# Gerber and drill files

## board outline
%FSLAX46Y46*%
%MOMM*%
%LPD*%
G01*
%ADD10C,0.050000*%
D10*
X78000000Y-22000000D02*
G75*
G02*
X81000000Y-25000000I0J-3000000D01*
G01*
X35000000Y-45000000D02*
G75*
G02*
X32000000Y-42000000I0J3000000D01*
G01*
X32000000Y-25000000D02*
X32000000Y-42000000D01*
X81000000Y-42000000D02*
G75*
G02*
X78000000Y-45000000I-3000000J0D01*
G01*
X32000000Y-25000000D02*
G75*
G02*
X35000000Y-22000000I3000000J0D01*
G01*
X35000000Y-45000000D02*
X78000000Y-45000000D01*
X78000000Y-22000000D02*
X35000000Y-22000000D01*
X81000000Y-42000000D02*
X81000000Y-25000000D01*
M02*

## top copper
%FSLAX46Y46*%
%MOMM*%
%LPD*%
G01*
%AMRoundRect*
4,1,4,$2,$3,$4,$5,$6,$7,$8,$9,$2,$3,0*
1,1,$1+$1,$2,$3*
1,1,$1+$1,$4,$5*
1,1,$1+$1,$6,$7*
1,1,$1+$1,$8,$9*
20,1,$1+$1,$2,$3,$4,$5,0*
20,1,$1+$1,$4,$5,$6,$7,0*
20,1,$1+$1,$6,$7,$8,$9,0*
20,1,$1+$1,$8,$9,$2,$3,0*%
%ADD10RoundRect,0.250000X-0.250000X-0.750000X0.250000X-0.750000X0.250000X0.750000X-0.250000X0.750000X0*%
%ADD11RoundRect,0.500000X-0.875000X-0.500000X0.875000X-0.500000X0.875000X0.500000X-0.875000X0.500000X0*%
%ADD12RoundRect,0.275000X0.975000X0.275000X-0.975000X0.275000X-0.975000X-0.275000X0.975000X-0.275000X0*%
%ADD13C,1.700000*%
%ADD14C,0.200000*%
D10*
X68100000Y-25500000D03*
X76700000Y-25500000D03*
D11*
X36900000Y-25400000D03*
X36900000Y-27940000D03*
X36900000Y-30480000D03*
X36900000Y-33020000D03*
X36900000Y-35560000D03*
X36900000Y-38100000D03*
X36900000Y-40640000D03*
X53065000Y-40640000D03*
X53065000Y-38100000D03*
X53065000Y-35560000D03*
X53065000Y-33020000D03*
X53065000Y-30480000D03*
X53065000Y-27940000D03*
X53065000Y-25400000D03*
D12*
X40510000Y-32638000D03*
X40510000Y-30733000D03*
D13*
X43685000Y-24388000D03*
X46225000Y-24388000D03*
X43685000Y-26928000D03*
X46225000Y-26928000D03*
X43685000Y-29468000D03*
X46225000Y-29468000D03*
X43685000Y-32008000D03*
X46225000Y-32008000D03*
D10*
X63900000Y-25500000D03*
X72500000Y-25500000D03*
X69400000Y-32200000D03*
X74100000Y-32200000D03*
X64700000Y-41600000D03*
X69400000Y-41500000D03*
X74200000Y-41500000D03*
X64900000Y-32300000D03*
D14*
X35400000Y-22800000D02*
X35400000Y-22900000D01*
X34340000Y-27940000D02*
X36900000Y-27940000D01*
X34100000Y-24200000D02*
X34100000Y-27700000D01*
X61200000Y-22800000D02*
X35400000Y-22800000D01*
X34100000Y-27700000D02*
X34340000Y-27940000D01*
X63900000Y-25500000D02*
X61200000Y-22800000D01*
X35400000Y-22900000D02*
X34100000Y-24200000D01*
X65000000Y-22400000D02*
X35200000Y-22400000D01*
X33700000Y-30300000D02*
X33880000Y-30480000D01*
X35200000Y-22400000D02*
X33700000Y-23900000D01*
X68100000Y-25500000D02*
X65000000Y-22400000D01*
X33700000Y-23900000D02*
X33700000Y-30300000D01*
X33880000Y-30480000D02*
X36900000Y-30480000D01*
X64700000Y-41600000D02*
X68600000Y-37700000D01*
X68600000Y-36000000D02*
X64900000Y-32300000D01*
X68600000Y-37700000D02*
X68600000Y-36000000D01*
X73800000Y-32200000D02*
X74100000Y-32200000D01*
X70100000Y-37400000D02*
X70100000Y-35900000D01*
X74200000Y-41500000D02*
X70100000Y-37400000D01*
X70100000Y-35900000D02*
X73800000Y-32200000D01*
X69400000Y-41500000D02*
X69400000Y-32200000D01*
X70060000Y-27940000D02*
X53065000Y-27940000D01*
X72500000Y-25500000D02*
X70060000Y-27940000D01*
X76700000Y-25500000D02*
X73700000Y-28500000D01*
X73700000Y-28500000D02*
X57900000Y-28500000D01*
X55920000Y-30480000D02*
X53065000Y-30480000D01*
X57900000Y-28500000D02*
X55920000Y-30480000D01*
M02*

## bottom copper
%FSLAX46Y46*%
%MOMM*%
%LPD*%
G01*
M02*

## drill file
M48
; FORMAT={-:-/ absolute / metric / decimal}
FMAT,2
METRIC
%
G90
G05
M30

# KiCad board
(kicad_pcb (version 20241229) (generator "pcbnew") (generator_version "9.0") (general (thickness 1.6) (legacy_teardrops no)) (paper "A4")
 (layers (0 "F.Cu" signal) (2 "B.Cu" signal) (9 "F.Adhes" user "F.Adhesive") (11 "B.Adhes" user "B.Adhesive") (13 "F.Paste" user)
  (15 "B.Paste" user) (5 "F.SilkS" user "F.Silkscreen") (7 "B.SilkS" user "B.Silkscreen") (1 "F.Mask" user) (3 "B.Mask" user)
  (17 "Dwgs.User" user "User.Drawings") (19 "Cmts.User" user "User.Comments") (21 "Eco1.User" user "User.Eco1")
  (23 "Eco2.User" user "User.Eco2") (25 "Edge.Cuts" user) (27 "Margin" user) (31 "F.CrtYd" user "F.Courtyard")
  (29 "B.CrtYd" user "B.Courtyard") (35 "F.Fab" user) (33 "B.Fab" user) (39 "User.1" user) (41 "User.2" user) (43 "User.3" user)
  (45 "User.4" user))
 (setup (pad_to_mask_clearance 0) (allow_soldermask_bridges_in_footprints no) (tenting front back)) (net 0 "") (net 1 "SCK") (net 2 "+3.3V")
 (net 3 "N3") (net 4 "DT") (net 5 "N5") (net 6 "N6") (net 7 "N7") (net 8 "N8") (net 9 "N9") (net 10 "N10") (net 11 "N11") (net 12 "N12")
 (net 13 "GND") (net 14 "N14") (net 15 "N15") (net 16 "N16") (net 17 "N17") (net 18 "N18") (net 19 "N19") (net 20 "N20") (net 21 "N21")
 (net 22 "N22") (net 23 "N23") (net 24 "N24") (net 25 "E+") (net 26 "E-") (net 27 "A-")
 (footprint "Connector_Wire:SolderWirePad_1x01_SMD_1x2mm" (layer "F.Cu") (at 68.1 25.5)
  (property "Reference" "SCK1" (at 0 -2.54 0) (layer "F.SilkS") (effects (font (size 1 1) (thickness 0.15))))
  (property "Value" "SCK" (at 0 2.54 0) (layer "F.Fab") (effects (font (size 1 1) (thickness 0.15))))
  (pad "1" smd roundrect (at 0 0) (size 1 2) (layers "F.Cu" "F.Mask" "F.Paste") (roundrect_rratio 0.25) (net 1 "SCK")))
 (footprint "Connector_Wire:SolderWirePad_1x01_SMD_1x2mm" (layer "F.Cu") (at 76.7 25.5)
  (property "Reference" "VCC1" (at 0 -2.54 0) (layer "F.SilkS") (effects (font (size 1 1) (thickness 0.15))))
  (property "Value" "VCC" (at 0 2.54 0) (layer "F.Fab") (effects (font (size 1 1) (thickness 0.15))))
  (pad "1" smd roundrect (at 0 0) (size 1 2) (layers "F.Cu" "F.Mask" "F.Paste") (roundrect_rratio 0.25) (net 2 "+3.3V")))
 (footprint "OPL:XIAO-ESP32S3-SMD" (layer "F.Cu") (at 44.961364 32.973)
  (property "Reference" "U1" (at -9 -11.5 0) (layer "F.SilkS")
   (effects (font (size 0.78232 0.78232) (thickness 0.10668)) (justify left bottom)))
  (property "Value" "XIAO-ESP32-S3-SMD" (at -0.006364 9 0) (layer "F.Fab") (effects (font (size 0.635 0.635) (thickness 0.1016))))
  (pad "1" smd roundrect (at -8.061364 -7.573) (size 2.75 2) (layers "F.Cu" "F.Mask" "F.Paste") (roundrect_rratio 0.25) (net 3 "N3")
   (solder_mask_margin 0.0508) (thermal_bridge_angle 45))
  (pad "2" smd roundrect (at -8.061364 -5.033) (size 2.75 2) (layers "F.Cu" "F.Mask" "F.Paste") (roundrect_rratio 0.25) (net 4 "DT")
   (solder_mask_margin 0.0508) (thermal_bridge_angle 45))
  (pad "3" smd roundrect (at -8.061364 -2.493) (size 2.75 2) (layers "F.Cu" "F.Mask" "F.Paste") (roundrect_rratio 0.25) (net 1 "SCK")
   (solder_mask_margin 0.0508) (thermal_bridge_angle 45))
  (pad "4" smd roundrect (at -8.061364 0.047) (size 2.75 2) (layers "F.Cu" "F.Mask" "F.Paste") (roundrect_rratio 0.25) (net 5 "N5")
   (solder_mask_margin 0.0508) (thermal_bridge_angle 45))
  (pad "5" smd roundrect (at -8.061364 2.587) (size 2.75 2) (layers "F.Cu" "F.Mask" "F.Paste") (roundrect_rratio 0.25) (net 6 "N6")
   (solder_mask_margin 0.0508) (thermal_bridge_angle 45))
  (pad "6" smd roundrect (at -8.061364 5.127) (size 2.75 2) (layers "F.Cu" "F.Mask" "F.Paste") (roundrect_rratio 0.25) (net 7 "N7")
   (solder_mask_margin 0.0508) (thermal_bridge_angle 45))
  (pad "7" smd roundrect (at -8.061364 7.667) (size 2.75 2) (layers "F.Cu" "F.Mask" "F.Paste") (roundrect_rratio 0.25) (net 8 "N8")
   (solder_mask_margin 0.0508) (thermal_bridge_angle 45))
  (pad "8" smd roundrect (at 8.103636 7.667) (size 2.75 2) (layers "F.Cu" "F.Mask" "F.Paste") (roundrect_rratio 0.25) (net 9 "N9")
   (solder_mask_margin 0.0508) (thermal_bridge_angle 45))
  (pad "9" smd roundrect (at 8.103636 5.127) (size 2.75 2) (layers "F.Cu" "F.Mask" "F.Paste") (roundrect_rratio 0.25) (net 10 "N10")
   (solder_mask_margin 0.0508) (thermal_bridge_angle 45))
  (pad "10" smd roundrect (at 8.103636 2.587) (size 2.75 2) (layers "F.Cu" "F.Mask" "F.Paste") (roundrect_rratio 0.25) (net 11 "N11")
   (solder_mask_margin 0.0508) (thermal_bridge_angle 45))
  (pad "11" smd roundrect (at 8.103636 0.047) (size 2.75 2) (layers "F.Cu" "F.Mask" "F.Paste") (roundrect_rratio 0.25) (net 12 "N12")
   (solder_mask_margin 0.0508) (thermal_bridge_angle 45))
  (pad "12" smd roundrect (at 8.103636 -2.493) (size 2.75 2) (layers "F.Cu" "F.Mask" "F.Paste") (roundrect_rratio 0.25) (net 2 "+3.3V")
   (solder_mask_margin 0.0508) (thermal_bridge_angle 45))
  (pad "13" smd roundrect (at 8.103636 -5.033) (size 2.75 2) (layers "F.Cu" "F.Mask" "F.Paste") (roundrect_rratio 0.25) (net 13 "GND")
   (solder_mask_margin 0.0508) (thermal_bridge_angle 45))
  (pad "14" smd roundrect (at 8.103636 -7.573) (size 2.75 2) (layers "F.Cu" "F.Mask" "F.Paste") (roundrect_rratio 0.25) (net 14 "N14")
   (solder_mask_margin 0.0508) (thermal_bridge_angle 45))
  (pad "15" smd roundrect (at -4.451364 -0.335 180) (size 2.5 1.1) (layers "F.Cu" "F.Mask" "F.Paste") (roundrect_rratio 0.25) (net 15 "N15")
   (solder_mask_margin 0.0508) (thermal_bridge_angle 45))
  (pad "16" smd roundrect (at -4.451364 -2.24 180) (size 2.5 1.1) (layers "F.Cu" "F.Mask" "F.Paste") (roundrect_rratio 0.25) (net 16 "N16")
   (solder_mask_margin 0.0508) (thermal_bridge_angle 45))
  (pad "17" smd circle (at -1.276364 -8.585) (size 1.7 1.7) (layers "F.Cu" "F.Mask" "F.Paste") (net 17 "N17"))
  (pad "18" smd circle (at 1.263636 -8.585) (size 1.7 1.7) (layers "F.Cu" "F.Mask" "F.Paste") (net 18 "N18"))
  (pad "19" smd circle (at -1.276364 -6.045) (size 1.7 1.7) (layers "F.Cu" "F.Mask" "F.Paste") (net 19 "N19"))
  (pad "20" smd circle (at 1.263636 -6.045) (size 1.7 1.7) (layers "F.Cu" "F.Mask" "F.Paste") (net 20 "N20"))
  (pad "21" smd circle (at -1.276364 -3.505) (size 1.7 1.7) (layers "F.Cu" "F.Mask" "F.Paste") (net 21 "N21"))
  (pad "22" smd circle (at 1.263636 -3.505) (size 1.7 1.7) (layers "F.Cu" "F.Mask" "F.Paste") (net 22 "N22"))
  (pad "23" smd circle (at -1.276364 -0.965) (size 1.7 1.7) (layers "F.Cu" "F.Mask" "F.Paste") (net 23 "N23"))
  (pad "24" smd circle (at 1.263636 -0.965) (size 1.7 1.7) (layers "F.Cu" "F.Mask" "F.Paste") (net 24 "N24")))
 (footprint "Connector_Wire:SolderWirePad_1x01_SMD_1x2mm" (layer "F.Cu") (at 63.9 25.5)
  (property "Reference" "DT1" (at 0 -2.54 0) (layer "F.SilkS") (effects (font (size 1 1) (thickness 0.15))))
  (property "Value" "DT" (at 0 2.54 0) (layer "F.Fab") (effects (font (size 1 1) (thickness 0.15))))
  (pad "1" smd roundrect (at 0 0) (size 1 2) (layers "F.Cu" "F.Mask" "F.Paste") (roundrect_rratio 0.25) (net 4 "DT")))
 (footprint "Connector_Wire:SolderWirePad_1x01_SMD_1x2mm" (layer "F.Cu") (at 72.5 25.5)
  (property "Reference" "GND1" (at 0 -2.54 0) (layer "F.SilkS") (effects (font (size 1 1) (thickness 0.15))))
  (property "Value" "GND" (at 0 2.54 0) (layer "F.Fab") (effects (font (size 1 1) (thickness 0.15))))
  (pad "1" smd roundrect (at 0 0) (size 1 2) (layers "F.Cu" "F.Mask" "F.Paste") (roundrect_rratio 0.25) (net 13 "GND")))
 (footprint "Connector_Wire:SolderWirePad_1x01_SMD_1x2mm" (layer "F.Cu") (at 69.4 32.2)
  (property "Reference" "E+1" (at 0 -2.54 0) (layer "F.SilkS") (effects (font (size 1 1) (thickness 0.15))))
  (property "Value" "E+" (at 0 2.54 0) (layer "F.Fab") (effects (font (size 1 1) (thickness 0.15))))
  (pad "1" smd roundrect (at 0 0) (size 1 2) (layers "F.Cu" "F.Mask" "F.Paste") (roundrect_rratio 0.25) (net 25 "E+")))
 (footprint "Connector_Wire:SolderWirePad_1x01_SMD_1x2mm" (layer "F.Cu") (at 74.1 32.2)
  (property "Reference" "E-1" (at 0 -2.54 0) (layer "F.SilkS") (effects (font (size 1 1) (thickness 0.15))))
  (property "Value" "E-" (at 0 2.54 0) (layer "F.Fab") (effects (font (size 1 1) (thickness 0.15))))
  (pad "1" smd roundrect (at 0 0) (size 1 2) (layers "F.Cu" "F.Mask" "F.Paste") (roundrect_rratio 0.25) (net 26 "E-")))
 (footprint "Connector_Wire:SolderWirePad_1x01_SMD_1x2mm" (layer "F.Cu") (at 64.7 41.6)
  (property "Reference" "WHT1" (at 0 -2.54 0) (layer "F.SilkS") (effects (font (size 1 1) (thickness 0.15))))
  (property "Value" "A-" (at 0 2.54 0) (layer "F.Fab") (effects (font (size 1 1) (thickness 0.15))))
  (pad "1" smd roundrect (at 0 0) (size 1 2) (layers "F.Cu" "F.Mask" "F.Paste") (roundrect_rratio 0.25) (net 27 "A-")))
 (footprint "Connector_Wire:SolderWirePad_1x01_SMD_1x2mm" (layer "F.Cu") (at 69.4 41.5)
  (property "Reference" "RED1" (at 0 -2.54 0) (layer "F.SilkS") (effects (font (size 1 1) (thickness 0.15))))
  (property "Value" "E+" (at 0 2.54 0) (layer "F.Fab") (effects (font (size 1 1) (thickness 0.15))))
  (pad "1" smd roundrect (at 0 0) (size 1 2) (layers "F.Cu" "F.Mask" "F.Paste") (roundrect_rratio 0.25) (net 25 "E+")))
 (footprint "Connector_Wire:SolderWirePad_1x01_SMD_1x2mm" (layer "F.Cu") (at 74.2 41.5)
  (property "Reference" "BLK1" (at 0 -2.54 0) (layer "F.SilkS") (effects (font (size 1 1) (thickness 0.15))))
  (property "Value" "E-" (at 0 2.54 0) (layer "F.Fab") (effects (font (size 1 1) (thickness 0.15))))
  (pad "1" smd roundrect (at 0 0) (size 1 2) (layers "F.Cu" "F.Mask" "F.Paste") (roundrect_rratio 0.25) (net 26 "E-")))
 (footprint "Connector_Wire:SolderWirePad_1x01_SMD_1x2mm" (layer "F.Cu") (at 64.9 32.3)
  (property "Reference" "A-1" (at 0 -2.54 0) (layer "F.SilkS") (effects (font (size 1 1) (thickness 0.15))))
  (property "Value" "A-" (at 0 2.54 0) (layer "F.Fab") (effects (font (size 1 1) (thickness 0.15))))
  (pad "1" smd roundrect (at 0 0) (size 1 2) (layers "F.Cu" "F.Mask" "F.Paste") (roundrect_rratio 0.25) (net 27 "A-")))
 (gr_arc (start 78 22) (mid 80.12132 22.87868) (end 81 25) (stroke (width 0.05) (type default)) (layer "Edge.Cuts"))
 (gr_arc (start 35 45) (mid 32.87868 44.12132) (end 32 42) (stroke (width 0.05) (type default)) (layer "Edge.Cuts"))
 (gr_line (start 32 25) (end 32 42) (stroke (width 0.05) (type default)) (layer "Edge.Cuts"))
 (gr_arc (start 81 42) (mid 80.12132 44.12132) (end 78 45) (stroke (width 0.05) (type default)) (layer "Edge.Cuts"))
 (gr_arc (start 32 25) (mid 32.87868 22.87868) (end 35 22) (stroke (width 0.05) (type default)) (layer "Edge.Cuts"))
 (gr_line (start 35 45) (end 78 45) (stroke (width 0.05) (type default)) (layer "Edge.Cuts"))
 (gr_line (start 78 22) (end 35 22) (stroke (width 0.05) (type default)) (layer "Edge.Cuts"))
 (gr_line (start 81 42) (end 81 25) (stroke (width 0.05) (type default)) (layer "Edge.Cuts"))
 (segment (start 35.4 22.8) (end 35.4 22.9) (width 0.2) (layer "F.Cu") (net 4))
 (segment (start 34.34 27.94) (end 36.9 27.94) (width 0.2) (layer "F.Cu") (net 4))
 (segment (start 34.1 24.2) (end 34.1 27.7) (width 0.2) (layer "F.Cu") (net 4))
 (segment (start 61.2 22.8) (end 35.4 22.8) (width 0.2) (layer "F.Cu") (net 4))
 (segment (start 34.1 27.7) (end 34.34 27.94) (width 0.2) (layer "F.Cu") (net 4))
 (segment (start 63.9 25.5) (end 61.2 22.8) (width 0.2) (layer "F.Cu") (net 4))
 (segment (start 35.4 22.9) (end 34.1 24.2) (width 0.2) (layer "F.Cu") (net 4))
 (segment (start 65 22.4) (end 35.2 22.4) (width 0.2) (layer "F.Cu") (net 1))
 (segment (start 33.7 30.3) (end 33.88 30.48) (width 0.2) (layer "F.Cu") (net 1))
 (segment (start 35.2 22.4) (end 33.7 23.9) (width 0.2) (layer "F.Cu") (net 1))
 (segment (start 68.1 25.5) (end 65 22.4) (width 0.2) (layer "F.Cu") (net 1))
 (segment (start 33.7 23.9) (end 33.7 30.3) (width 0.2) (layer "F.Cu") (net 1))
 (segment (start 33.88 30.48) (end 36.9 30.48) (width 0.2) (layer "F.Cu") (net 1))
 (segment (start 64.7 41.6) (end 68.6 37.7) (width 0.2) (layer "F.Cu") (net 27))
 (segment (start 68.6 36) (end 64.9 32.3) (width 0.2) (layer "F.Cu") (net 27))
 (segment (start 68.6 37.7) (end 68.6 36) (width 0.2) (layer "F.Cu") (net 27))
 (segment (start 73.8 32.2) (end 74.1 32.2) (width 0.2) (layer "F.Cu") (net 26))
 (segment (start 70.1 37.4) (end 70.1 35.9) (width 0.2) (layer "F.Cu") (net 26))
 (segment (start 74.2 41.5) (end 70.1 37.4) (width 0.2) (layer "F.Cu") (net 26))
 (segment (start 70.1 35.9) (end 73.8 32.2) (width 0.2) (layer "F.Cu") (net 26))
 (segment (start 69.4 41.5) (end 69.4 32.2) (width 0.2) (layer "F.Cu") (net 25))
 (segment (start 70.06 27.94) (end 53.065 27.94) (width 0.2) (layer "F.Cu") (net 13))
 (segment (start 72.5 25.5) (end 70.06 27.94) (width 0.2) (layer "F.Cu") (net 13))
 (segment (start 76.7 25.5) (end 73.7 28.5) (width 0.2) (layer "F.Cu") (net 2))
 (segment (start 73.7 28.5) (end 57.9 28.5) (width 0.2) (layer "F.Cu") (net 2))
 (segment (start 55.92 30.48) (end 53.065 30.48) (width 0.2) (layer "F.Cu") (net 2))
 (segment (start 57.9 28.5) (end 55.92 30.48) (width 0.2) (layer "F.Cu") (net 2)))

